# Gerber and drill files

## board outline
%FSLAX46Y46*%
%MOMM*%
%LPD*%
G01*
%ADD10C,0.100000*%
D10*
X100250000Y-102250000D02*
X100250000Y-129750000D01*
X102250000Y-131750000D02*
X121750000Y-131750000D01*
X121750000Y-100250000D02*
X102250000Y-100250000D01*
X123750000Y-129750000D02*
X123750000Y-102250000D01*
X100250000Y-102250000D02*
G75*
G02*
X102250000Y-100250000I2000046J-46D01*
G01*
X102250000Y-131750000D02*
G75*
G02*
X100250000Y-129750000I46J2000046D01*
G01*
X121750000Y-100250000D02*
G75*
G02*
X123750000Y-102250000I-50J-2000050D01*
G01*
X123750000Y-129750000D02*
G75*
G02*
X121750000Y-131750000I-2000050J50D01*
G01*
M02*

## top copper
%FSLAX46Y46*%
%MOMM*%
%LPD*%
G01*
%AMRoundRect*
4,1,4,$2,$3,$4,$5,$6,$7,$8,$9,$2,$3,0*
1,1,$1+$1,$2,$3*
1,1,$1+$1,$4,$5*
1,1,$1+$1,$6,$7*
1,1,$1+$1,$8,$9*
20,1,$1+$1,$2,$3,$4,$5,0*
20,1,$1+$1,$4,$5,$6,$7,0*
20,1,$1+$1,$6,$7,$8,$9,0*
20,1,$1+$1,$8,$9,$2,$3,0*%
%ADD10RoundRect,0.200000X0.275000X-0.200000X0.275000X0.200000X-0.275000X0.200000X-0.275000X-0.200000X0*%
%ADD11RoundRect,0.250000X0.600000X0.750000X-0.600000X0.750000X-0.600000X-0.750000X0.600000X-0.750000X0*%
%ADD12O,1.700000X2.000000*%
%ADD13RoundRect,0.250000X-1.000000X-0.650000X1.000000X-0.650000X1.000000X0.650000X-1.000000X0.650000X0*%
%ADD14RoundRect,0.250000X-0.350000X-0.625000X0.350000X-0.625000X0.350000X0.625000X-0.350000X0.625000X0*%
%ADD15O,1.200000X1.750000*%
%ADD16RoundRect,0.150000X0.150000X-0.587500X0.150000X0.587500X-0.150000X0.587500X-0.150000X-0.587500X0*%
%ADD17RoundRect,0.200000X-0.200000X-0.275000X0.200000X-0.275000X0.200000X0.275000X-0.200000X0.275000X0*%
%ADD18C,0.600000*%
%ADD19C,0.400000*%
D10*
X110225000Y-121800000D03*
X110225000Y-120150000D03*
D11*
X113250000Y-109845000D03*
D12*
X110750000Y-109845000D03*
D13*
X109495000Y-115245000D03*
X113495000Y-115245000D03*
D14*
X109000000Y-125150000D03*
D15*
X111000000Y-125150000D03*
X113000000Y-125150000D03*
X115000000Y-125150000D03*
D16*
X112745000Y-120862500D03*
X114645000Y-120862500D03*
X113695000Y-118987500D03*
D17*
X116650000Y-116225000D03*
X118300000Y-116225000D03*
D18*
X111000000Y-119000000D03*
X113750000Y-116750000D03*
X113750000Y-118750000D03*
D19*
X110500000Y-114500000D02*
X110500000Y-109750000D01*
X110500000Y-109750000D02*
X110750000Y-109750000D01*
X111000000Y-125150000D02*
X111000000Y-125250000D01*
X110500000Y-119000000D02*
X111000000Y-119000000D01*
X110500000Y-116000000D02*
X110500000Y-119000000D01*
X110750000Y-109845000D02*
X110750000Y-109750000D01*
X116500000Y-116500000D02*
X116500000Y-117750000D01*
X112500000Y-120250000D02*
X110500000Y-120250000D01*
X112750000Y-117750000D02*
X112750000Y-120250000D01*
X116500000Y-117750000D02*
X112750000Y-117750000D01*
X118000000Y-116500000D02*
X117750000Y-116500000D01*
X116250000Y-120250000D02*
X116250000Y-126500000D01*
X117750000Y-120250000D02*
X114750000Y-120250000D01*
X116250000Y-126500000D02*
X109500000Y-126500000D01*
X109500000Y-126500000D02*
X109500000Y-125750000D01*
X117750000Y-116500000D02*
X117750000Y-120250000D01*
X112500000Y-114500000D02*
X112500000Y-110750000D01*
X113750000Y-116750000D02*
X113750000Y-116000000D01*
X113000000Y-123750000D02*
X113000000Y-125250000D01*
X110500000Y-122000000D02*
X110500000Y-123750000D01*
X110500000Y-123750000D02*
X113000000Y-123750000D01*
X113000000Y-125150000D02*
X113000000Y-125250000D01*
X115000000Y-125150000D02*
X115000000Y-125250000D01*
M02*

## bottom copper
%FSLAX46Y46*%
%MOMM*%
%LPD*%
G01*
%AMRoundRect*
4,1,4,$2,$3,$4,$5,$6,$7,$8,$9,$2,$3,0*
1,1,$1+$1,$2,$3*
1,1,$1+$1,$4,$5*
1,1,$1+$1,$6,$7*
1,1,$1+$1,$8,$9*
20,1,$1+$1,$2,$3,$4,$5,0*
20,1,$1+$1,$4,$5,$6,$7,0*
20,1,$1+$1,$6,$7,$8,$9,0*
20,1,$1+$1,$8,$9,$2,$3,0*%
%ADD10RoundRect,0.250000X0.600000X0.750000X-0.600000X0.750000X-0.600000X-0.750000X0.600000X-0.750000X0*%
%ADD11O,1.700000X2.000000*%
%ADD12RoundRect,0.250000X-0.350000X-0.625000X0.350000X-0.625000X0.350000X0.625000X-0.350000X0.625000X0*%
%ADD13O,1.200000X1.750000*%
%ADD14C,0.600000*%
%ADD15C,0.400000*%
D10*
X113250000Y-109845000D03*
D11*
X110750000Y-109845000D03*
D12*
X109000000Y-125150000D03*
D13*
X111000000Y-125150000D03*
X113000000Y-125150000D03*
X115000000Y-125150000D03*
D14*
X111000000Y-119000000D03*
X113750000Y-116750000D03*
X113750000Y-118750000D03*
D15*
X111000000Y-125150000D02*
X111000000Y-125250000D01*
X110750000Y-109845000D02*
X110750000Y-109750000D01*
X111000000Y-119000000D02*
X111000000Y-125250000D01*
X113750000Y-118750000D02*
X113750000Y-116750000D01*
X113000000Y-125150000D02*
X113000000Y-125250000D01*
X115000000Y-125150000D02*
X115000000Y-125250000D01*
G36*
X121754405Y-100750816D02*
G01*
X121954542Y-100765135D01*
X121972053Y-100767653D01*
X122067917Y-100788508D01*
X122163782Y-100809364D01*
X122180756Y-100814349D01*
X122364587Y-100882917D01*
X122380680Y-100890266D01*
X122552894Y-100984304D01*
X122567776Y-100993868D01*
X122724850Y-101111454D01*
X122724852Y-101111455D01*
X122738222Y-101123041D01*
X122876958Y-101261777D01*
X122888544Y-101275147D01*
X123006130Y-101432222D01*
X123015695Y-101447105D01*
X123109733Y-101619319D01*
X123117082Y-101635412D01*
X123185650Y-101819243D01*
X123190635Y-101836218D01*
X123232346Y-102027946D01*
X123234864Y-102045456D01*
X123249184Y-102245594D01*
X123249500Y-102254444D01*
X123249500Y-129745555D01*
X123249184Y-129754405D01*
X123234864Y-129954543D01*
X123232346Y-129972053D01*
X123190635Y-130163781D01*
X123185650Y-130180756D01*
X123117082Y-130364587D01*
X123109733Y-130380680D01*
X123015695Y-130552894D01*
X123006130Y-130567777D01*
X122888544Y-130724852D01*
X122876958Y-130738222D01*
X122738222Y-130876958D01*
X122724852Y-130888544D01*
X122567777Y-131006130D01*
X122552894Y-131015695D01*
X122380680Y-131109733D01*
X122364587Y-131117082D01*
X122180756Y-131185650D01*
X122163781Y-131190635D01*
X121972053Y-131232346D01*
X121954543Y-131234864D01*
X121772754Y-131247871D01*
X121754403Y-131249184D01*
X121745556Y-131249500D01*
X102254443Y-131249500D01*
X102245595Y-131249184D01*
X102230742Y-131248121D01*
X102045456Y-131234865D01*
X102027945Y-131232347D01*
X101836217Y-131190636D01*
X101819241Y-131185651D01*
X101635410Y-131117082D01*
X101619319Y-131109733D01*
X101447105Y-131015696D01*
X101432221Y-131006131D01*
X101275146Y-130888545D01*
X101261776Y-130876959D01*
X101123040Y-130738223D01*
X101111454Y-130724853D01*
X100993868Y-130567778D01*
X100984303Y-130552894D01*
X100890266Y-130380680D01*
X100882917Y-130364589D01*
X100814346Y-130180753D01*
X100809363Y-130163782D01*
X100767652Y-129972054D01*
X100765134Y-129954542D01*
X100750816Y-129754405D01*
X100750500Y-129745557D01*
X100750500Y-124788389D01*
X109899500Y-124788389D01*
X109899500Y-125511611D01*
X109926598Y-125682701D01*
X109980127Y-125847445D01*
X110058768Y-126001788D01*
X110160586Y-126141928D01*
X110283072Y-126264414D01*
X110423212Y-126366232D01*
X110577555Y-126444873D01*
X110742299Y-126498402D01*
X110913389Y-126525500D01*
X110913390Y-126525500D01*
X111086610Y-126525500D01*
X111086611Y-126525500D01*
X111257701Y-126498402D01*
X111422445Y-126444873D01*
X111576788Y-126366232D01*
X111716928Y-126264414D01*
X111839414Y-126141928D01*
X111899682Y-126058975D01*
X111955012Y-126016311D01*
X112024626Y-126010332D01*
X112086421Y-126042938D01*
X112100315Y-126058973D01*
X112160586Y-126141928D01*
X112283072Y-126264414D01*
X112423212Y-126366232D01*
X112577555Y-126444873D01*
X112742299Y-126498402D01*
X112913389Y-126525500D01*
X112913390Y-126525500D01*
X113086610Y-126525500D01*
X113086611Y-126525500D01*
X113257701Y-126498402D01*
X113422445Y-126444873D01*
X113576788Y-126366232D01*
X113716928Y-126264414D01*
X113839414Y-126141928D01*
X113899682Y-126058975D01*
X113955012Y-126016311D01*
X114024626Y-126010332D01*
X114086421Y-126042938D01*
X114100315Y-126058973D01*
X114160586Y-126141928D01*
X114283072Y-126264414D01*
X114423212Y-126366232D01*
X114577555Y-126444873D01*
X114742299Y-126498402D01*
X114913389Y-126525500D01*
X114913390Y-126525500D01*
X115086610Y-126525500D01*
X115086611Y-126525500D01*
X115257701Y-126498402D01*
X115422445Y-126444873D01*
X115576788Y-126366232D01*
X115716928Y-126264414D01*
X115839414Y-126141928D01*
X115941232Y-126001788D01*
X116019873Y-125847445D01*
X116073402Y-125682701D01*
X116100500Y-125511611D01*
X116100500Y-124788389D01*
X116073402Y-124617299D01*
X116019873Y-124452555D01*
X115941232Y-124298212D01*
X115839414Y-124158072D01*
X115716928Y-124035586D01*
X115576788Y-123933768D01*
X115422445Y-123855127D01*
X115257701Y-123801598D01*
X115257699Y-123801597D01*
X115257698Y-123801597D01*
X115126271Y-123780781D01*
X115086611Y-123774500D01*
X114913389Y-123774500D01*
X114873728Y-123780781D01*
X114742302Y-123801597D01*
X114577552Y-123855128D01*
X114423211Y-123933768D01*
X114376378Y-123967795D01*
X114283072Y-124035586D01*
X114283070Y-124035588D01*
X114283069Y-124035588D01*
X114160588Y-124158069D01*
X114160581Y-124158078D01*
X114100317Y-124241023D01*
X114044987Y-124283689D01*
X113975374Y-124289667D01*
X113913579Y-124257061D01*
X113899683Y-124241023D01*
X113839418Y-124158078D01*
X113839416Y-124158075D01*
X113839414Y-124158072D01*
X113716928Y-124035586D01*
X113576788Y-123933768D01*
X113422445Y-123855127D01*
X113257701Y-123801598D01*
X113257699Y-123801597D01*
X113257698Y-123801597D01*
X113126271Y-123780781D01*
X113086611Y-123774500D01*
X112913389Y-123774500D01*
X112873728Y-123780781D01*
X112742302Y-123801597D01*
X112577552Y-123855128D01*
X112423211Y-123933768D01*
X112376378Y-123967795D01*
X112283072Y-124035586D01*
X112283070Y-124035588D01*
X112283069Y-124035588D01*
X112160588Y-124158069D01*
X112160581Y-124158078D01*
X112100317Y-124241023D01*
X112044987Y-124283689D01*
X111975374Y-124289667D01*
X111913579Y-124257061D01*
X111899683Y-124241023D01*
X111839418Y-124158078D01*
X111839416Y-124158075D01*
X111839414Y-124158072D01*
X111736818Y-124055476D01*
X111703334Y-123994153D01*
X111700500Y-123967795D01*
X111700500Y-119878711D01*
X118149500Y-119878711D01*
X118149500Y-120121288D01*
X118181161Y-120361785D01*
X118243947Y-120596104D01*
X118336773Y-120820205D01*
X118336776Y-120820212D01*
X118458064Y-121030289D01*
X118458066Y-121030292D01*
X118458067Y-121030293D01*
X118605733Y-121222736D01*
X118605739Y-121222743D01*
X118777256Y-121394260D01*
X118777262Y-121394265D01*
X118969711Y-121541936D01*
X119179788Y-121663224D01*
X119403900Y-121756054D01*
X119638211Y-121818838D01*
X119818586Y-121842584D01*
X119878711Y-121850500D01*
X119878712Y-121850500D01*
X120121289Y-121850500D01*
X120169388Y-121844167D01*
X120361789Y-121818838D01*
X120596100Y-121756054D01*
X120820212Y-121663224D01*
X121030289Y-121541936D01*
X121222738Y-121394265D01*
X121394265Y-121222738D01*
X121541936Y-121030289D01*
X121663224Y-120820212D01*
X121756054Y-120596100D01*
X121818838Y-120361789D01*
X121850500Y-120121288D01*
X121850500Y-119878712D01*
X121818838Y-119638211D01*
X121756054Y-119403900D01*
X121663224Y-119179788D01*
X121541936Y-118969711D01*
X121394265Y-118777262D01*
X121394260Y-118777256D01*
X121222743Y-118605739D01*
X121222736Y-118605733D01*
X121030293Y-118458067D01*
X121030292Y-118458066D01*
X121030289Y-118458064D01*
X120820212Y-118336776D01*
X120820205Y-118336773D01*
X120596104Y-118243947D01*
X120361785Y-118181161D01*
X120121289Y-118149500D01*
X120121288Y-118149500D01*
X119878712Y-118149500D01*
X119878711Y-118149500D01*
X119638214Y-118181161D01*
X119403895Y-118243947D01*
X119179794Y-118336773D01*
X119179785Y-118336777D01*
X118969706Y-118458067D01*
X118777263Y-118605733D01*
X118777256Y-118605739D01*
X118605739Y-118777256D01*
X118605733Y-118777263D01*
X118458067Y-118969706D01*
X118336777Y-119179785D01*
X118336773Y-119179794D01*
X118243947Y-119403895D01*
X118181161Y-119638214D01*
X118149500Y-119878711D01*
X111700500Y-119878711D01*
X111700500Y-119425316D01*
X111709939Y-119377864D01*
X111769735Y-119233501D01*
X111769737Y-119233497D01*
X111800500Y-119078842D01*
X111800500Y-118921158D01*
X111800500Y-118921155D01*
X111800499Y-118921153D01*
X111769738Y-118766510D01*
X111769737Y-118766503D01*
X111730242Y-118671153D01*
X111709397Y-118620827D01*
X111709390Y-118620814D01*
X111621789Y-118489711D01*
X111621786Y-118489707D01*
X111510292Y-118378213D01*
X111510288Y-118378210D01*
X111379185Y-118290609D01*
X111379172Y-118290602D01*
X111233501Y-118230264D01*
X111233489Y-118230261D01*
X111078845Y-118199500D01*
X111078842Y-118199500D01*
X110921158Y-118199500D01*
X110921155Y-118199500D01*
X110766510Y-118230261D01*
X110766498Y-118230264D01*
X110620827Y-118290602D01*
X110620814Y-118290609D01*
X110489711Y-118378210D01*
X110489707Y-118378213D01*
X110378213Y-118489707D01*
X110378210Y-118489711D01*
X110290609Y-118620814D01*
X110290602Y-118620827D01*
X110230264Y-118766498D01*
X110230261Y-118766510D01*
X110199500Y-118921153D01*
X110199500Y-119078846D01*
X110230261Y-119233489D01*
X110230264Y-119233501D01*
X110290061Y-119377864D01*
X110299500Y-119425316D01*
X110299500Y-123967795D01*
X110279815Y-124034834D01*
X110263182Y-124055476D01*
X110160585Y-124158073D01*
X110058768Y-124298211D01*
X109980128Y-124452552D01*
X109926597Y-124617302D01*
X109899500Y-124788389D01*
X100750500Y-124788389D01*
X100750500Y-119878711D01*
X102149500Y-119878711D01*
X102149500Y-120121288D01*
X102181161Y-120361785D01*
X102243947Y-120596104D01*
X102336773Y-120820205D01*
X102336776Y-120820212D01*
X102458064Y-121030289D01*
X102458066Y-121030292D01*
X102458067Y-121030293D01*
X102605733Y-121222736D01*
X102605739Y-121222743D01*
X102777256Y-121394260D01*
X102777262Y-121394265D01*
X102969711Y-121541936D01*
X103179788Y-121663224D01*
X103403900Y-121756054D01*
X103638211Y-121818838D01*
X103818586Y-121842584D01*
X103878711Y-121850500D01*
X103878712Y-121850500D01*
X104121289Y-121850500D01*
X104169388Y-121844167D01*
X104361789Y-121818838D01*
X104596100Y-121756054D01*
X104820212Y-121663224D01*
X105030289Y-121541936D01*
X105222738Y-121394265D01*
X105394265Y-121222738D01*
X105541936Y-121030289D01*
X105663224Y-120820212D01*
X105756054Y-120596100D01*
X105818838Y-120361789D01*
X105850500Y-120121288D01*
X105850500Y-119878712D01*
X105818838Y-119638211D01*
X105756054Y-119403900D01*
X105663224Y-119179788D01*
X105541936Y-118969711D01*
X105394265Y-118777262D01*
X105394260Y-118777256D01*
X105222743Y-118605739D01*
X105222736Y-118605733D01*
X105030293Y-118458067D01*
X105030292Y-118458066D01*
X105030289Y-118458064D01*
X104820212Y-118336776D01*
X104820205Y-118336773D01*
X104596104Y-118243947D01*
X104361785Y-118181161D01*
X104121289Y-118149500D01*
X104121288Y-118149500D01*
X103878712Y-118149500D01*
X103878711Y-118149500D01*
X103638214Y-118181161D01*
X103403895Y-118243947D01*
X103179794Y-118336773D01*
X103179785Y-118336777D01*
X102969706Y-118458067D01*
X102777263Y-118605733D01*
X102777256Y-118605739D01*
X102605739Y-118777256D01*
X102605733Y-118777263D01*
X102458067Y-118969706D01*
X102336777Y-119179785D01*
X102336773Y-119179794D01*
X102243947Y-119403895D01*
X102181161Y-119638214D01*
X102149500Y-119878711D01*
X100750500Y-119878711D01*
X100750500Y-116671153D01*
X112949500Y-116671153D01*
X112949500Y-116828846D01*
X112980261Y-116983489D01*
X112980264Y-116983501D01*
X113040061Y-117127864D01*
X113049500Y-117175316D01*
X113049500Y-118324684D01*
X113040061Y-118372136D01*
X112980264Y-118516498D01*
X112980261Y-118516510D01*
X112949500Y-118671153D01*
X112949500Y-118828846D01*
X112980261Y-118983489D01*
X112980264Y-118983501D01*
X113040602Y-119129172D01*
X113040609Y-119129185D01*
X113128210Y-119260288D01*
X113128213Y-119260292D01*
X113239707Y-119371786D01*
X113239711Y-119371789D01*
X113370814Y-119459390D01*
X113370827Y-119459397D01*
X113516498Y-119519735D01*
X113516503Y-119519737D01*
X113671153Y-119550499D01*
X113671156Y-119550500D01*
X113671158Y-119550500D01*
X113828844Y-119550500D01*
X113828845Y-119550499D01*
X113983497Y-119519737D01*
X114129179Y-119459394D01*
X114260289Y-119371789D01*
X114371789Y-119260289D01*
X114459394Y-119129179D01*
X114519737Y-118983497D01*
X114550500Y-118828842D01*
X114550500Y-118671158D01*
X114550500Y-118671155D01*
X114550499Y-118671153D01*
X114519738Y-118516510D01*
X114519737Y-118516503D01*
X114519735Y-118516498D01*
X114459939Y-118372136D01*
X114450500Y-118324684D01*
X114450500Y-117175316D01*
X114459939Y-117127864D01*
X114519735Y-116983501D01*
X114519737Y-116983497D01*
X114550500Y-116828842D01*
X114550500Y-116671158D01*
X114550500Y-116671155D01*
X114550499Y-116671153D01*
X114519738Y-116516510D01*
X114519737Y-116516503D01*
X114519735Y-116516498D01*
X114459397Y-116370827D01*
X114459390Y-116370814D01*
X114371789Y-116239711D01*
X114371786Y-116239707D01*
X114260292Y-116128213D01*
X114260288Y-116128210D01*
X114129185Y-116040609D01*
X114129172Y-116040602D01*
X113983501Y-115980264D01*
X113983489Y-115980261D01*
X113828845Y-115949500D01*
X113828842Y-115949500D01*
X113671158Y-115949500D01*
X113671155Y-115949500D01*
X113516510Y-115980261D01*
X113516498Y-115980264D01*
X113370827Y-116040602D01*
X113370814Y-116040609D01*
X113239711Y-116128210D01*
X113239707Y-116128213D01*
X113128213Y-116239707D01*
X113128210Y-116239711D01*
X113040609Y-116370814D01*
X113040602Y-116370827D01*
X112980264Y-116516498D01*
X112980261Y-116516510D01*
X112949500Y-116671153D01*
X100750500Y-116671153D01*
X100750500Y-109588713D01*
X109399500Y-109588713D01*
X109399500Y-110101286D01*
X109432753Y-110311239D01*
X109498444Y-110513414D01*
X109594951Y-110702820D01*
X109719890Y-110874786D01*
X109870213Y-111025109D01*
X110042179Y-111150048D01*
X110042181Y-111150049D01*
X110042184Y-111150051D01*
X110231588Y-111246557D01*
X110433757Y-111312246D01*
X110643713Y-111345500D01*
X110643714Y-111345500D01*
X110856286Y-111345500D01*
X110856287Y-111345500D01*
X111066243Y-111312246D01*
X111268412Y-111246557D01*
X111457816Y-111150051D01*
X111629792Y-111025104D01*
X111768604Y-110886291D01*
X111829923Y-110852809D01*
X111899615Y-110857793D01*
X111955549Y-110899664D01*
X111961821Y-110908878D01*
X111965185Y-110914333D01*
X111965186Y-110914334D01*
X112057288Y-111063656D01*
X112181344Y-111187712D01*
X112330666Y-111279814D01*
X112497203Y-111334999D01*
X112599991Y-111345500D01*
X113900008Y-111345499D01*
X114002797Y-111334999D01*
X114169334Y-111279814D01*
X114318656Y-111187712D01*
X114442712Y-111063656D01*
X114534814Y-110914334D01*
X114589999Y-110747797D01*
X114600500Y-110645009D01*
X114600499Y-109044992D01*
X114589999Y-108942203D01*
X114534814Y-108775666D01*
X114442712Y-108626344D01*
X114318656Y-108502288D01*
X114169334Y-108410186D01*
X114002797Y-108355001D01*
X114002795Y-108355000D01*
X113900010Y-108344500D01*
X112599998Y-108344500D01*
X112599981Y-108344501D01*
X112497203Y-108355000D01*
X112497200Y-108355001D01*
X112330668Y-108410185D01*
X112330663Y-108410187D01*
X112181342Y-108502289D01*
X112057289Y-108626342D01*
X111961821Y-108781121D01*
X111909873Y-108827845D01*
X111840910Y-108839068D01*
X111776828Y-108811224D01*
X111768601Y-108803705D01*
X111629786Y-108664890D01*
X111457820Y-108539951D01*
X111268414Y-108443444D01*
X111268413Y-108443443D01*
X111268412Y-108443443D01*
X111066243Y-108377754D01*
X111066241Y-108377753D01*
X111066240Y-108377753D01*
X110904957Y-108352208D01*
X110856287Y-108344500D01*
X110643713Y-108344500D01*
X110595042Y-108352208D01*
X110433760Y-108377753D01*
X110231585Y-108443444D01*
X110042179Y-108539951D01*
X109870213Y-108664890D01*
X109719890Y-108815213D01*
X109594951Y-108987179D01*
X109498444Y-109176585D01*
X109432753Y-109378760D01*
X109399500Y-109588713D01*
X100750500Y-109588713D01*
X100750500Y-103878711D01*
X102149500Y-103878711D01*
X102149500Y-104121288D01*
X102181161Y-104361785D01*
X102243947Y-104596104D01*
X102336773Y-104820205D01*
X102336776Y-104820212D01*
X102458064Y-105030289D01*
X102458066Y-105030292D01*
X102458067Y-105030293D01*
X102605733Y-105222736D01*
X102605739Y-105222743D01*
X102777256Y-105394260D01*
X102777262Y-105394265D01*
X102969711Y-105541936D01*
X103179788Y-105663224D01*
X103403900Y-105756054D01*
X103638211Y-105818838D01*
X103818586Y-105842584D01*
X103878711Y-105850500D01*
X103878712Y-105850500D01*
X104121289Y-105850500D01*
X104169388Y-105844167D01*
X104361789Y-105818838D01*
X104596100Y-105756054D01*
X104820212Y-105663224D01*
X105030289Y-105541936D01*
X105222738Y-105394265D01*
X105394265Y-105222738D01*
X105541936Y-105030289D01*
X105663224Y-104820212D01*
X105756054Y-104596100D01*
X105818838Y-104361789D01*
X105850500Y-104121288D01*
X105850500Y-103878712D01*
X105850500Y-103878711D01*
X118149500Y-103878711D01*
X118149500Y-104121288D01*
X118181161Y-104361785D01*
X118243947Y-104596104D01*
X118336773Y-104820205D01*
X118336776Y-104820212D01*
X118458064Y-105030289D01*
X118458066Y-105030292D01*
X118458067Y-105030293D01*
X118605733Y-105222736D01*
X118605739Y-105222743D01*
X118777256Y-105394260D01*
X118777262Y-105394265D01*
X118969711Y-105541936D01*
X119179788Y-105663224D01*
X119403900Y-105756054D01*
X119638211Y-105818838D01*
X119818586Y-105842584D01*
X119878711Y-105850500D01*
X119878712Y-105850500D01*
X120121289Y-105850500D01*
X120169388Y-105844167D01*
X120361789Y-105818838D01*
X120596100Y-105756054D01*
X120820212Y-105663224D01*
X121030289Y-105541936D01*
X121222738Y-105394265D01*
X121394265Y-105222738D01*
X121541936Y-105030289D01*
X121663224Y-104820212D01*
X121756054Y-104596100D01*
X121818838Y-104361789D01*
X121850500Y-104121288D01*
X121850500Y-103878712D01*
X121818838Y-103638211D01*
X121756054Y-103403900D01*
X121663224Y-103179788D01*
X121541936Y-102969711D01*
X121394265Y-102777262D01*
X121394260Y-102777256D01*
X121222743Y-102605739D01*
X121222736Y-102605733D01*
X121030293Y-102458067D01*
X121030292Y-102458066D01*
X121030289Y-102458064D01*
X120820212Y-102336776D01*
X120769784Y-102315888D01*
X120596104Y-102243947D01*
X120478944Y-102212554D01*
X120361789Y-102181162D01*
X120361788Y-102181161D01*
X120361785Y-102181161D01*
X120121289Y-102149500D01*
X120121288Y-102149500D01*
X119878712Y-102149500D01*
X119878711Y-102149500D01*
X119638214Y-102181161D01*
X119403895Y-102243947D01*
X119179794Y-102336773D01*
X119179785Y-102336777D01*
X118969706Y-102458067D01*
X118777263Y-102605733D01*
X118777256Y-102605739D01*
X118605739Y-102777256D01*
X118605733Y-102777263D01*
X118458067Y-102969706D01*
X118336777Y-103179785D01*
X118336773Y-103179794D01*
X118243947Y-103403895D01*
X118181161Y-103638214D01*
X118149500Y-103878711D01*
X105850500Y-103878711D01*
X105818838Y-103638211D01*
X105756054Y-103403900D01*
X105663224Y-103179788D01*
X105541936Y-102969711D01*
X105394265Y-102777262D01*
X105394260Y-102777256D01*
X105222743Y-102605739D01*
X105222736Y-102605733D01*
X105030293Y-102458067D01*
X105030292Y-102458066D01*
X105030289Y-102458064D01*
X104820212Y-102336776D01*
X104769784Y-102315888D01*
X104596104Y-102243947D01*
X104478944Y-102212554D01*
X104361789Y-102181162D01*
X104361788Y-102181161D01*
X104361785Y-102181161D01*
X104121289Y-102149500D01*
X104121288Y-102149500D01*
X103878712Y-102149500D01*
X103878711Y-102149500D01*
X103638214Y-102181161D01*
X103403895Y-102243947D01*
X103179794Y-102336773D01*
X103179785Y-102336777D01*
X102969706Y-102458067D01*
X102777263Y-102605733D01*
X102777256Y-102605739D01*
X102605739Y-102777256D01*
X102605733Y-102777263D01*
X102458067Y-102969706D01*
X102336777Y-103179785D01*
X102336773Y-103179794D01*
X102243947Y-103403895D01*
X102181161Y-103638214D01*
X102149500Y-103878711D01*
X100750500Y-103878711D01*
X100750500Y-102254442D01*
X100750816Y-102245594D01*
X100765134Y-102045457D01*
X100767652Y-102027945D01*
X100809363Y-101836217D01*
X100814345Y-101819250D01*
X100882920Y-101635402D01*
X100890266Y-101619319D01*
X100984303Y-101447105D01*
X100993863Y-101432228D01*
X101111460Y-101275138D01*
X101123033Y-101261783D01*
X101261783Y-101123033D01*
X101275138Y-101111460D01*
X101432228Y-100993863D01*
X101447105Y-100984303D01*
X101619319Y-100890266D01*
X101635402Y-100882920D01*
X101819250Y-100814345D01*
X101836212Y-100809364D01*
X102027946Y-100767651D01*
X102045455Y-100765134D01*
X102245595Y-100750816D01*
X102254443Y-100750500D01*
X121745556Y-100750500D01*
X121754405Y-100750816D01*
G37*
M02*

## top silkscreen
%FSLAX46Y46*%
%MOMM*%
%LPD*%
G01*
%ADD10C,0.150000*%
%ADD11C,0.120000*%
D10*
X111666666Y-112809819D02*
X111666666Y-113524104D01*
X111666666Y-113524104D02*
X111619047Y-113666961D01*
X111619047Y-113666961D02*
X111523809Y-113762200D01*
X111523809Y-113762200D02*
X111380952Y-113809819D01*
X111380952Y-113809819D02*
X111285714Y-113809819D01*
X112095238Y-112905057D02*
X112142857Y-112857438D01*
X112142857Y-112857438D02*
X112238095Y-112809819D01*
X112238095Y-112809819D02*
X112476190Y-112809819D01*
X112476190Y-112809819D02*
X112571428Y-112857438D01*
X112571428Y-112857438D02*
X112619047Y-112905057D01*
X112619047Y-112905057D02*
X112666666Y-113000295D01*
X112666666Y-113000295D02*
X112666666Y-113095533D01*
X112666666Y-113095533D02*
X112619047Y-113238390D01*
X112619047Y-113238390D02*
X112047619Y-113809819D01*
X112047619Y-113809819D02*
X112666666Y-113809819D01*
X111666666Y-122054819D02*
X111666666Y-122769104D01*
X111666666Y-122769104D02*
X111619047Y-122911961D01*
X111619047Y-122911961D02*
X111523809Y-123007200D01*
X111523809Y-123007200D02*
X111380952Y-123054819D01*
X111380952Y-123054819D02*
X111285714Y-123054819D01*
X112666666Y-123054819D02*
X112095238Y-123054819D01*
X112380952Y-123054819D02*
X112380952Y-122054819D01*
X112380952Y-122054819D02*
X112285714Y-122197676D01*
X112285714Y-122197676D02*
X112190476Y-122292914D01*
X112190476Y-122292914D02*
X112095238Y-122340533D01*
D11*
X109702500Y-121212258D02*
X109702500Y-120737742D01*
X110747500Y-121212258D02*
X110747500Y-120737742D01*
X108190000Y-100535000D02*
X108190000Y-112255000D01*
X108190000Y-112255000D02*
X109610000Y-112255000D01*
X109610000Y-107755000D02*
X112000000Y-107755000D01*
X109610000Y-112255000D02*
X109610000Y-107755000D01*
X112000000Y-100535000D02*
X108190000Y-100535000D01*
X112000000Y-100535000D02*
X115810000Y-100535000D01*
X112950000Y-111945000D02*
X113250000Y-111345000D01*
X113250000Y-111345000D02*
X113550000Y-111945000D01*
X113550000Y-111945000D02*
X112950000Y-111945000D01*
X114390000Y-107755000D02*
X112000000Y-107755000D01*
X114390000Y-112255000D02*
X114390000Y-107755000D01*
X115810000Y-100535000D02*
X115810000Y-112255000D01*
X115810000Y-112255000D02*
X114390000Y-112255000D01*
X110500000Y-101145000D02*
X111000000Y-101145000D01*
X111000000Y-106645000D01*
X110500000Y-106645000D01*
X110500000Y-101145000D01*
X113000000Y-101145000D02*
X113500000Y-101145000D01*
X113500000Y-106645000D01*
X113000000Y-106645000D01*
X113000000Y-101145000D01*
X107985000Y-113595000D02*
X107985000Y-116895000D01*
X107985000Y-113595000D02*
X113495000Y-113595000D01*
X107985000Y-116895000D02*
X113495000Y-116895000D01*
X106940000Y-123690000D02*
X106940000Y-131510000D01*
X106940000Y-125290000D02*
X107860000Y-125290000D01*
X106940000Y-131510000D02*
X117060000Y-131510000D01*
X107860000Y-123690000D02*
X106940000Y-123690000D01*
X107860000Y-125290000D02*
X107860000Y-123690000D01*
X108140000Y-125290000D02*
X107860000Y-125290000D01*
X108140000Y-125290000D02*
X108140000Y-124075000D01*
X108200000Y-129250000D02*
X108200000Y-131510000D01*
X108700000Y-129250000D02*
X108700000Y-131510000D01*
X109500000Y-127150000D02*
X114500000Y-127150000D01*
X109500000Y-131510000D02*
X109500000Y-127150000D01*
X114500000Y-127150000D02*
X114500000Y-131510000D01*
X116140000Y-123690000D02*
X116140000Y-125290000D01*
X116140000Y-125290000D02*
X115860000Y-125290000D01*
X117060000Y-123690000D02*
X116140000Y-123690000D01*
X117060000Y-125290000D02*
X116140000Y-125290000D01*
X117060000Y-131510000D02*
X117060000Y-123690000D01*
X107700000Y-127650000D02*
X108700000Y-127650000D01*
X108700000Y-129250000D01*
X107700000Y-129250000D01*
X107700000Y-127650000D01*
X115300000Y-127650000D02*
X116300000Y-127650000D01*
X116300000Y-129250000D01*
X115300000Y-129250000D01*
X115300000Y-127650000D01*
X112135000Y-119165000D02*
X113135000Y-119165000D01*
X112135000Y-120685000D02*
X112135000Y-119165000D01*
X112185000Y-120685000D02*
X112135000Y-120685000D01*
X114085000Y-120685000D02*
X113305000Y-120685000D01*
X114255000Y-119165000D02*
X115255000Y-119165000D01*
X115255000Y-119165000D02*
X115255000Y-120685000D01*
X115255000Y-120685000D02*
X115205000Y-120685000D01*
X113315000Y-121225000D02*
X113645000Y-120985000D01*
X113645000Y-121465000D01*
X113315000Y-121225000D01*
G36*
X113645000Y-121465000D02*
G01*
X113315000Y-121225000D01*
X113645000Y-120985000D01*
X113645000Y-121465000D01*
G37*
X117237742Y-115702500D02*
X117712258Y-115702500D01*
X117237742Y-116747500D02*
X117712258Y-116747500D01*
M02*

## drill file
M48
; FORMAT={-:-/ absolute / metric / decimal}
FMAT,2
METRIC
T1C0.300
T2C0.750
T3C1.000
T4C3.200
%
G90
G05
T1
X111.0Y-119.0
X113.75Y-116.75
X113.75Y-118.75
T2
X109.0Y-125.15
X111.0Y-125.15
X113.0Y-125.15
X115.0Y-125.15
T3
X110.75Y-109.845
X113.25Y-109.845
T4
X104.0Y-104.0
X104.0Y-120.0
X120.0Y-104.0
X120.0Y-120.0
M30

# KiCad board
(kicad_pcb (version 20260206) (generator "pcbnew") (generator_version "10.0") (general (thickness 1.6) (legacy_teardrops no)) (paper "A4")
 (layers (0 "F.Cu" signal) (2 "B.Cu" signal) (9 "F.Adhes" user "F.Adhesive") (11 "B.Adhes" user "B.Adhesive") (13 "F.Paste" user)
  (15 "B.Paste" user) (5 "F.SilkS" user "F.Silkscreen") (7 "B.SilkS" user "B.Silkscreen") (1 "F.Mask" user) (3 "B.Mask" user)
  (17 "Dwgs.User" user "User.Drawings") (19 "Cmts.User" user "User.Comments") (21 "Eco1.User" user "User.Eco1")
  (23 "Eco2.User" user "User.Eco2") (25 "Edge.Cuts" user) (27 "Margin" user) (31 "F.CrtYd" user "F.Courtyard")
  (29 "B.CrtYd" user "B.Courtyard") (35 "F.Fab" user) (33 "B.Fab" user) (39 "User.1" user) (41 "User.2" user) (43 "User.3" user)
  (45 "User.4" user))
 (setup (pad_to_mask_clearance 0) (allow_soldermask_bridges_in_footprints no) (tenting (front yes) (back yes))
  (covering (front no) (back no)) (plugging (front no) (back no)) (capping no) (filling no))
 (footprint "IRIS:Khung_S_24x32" (layer "F.Cu") (at 100 132)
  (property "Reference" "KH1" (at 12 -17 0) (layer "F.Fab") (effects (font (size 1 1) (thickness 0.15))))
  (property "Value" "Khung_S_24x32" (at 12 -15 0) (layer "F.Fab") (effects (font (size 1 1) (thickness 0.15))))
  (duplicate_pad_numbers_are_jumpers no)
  (fp_line (start 0.25 -29.75) (end 0.25 -2.25) (stroke (width 0.1) (type solid)) (layer "Edge.Cuts"))
  (fp_line (start 2.25 -0.25) (end 21.75 -0.25) (stroke (width 0.1) (type solid)) (layer "Edge.Cuts"))
  (fp_line (start 21.75 -31.75) (end 2.25 -31.75) (stroke (width 0.1) (type solid)) (layer "Edge.Cuts"))
  (fp_line (start 23.75 -2.25) (end 23.75 -29.75) (stroke (width 0.1) (type solid)) (layer "Edge.Cuts"))
  (fp_arc (start 0.25 -29.75) (mid 0.8358 -31.1642) (end 2.25 -31.75) (stroke (width 0.1) (type solid)) (layer "Edge.Cuts"))
  (fp_arc (start 2.25 -0.25) (mid 0.8358 -0.8358) (end 0.25 -2.25) (stroke (width 0.1) (type solid)) (layer "Edge.Cuts"))
  (fp_arc (start 21.75 -31.75) (mid 23.164199 -31.164199) (end 23.75 -29.75) (stroke (width 0.1) (type solid)) (layer "Edge.Cuts"))
  (fp_arc (start 23.75 -2.25) (mid 23.164199 -0.835801) (end 21.75 -0.25) (stroke (width 0.1) (type solid)) (layer "Edge.Cuts"))
  (pad "" np_thru_hole circle (at 4 -28) (size 3.2 3.2) (drill 3.2) (layers "*.Cu" "*.Mask"))
  (pad "" np_thru_hole circle (at 4 -12) (size 3.2 3.2) (drill 3.2) (layers "*.Cu" "*.Mask"))
  (pad "" np_thru_hole circle (at 20 -28) (size 3.2 3.2) (drill 3.2) (layers "*.Cu" "*.Mask"))
  (pad "" np_thru_hole circle (at 20 -12) (size 3.2 3.2) (drill 3.2) (layers "*.Cu" "*.Mask")))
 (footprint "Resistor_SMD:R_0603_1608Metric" (layer "F.Cu") (at 110.225 120.975 90)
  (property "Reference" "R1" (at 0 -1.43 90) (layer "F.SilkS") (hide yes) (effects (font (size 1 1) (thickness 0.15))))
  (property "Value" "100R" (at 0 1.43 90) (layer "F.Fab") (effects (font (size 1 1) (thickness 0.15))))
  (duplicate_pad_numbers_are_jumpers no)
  (fp_line (start -0.237258 -0.5225) (end 0.237258 -0.5225) (stroke (width 0.12) (type solid)) (layer "F.SilkS"))
  (fp_line (start -0.237258 0.5225) (end 0.237258 0.5225) (stroke (width 0.12) (type solid)) (layer "F.SilkS"))
  (pad "1" smd roundrect (at -0.825 0 90) (size 0.8 0.95) (layers "F.Cu" "F.Mask" "F.Paste") (roundrect_rratio 0.25) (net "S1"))
  (pad "2" smd roundrect (at 0.825 0 90) (size 0.8 0.95) (layers "F.Cu" "F.Mask" "F.Paste") (roundrect_rratio 0.25) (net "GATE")))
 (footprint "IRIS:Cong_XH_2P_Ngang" (layer "F.Cu") (at 113.25 109.845 180)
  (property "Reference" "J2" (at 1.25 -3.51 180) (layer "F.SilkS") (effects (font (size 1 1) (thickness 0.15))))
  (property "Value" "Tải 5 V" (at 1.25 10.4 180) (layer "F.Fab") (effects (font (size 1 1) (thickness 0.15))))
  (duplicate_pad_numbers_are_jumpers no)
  (fp_line (start 5.06 9.31) (end 5.06 -2.41) (stroke (width 0.12) (type solid)) (layer "F.SilkS"))
  (fp_line (start 5.06 -2.41) (end 3.64 -2.41) (stroke (width 0.12) (type solid)) (layer "F.SilkS"))
  (fp_line (start 3.64 2.09) (end 1.25 2.09) (stroke (width 0.12) (type solid)) (layer "F.SilkS"))
  (fp_line (start 3.64 -2.41) (end 3.64 2.09) (stroke (width 0.12) (type solid)) (layer "F.SilkS"))
  (fp_line (start 1.25 9.31) (end 5.06 9.31) (stroke (width 0.12) (type solid)) (layer "F.SilkS"))
  (fp_line (start 1.25 9.31) (end -2.56 9.31) (stroke (width 0.12) (type solid)) (layer "F.SilkS"))
  (fp_line (start 0.3 -2.1) (end 0 -1.5) (stroke (width 0.12) (type solid)) (layer "F.SilkS"))
  (fp_line (start 0 -1.5) (end -0.3 -2.1) (stroke (width 0.12) (type solid)) (layer "F.SilkS"))
  (fp_line (start -0.3 -2.1) (end 0.3 -2.1) (stroke (width 0.12) (type solid)) (layer "F.SilkS"))
  (fp_line (start -1.14 2.09) (end 1.25 2.09) (stroke (width 0.12) (type solid)) (layer "F.SilkS"))
  (fp_line (start -1.14 -2.41) (end -1.14 2.09) (stroke (width 0.12) (type solid)) (layer "F.SilkS"))
  (fp_line (start -2.56 9.31) (end -2.56 -2.41) (stroke (width 0.12) (type solid)) (layer "F.SilkS"))
  (fp_line (start -2.56 -2.41) (end -1.14 -2.41) (stroke (width 0.12) (type solid)) (layer "F.SilkS"))
  (fp_rect (start 2.25 3.2) (end 2.75 8.7) (stroke (width 0.12) (type solid)) (fill no) (layer "F.SilkS"))
  (fp_rect (start -0.25 3.2) (end 0.25 8.7) (stroke (width 0.12) (type solid)) (fill no) (layer "F.SilkS"))
  (pad "1" thru_hole roundrect (at 0 0 180) (size 1.7 2) (drill 1) (layers "*.Cu" "*.Mask") (remove_unused_layers no)
   (roundrect_rratio 0.147059) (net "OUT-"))
  (pad "2" thru_hole oval (at 2.5 0 180) (size 1.7 2) (drill 1) (layers "*.Cu" "*.Mask") (remove_unused_layers no) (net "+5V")))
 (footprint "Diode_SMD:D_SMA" (layer "F.Cu") (at 111.495 115.245)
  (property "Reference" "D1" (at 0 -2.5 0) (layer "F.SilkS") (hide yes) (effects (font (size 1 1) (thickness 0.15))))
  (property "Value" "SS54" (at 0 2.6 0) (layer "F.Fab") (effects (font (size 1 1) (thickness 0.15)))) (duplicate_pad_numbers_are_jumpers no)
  (fp_line (start -3.51 -1.65) (end -3.51 1.65) (stroke (width 0.12) (type solid)) (layer "F.SilkS"))
  (fp_line (start -3.51 -1.65) (end 2 -1.65) (stroke (width 0.12) (type solid)) (layer "F.SilkS"))
  (fp_line (start -3.51 1.65) (end 2 1.65) (stroke (width 0.12) (type solid)) (layer "F.SilkS"))
  (pad "1" smd roundrect (at -2 0) (size 2.5 1.8) (layers "F.Cu" "F.Mask" "F.Paste") (roundrect_rratio 0.1388888889) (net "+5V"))
  (pad "2" smd roundrect (at 2 0) (size 2.5 1.8) (layers "F.Cu" "F.Mask" "F.Paste") (roundrect_rratio 0.1388888889) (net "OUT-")))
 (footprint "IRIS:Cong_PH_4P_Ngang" (layer "F.Cu") (at 109 125.15)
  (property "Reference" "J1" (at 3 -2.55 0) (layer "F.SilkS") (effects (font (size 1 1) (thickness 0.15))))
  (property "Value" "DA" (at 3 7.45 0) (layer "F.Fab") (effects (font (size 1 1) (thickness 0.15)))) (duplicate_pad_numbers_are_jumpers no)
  (fp_line (start -2.06 -1.46) (end -2.06 6.36) (stroke (width 0.12) (type solid)) (layer "F.SilkS"))
  (fp_line (start -2.06 0.14) (end -1.14 0.14) (stroke (width 0.12) (type solid)) (layer "F.SilkS"))
  (fp_line (start -2.06 6.36) (end 8.06 6.36) (stroke (width 0.12) (type solid)) (layer "F.SilkS"))
  (fp_line (start -1.14 -1.46) (end -2.06 -1.46) (stroke (width 0.12) (type solid)) (layer "F.SilkS"))
  (fp_line (start -1.14 0.14) (end -1.14 -1.46) (stroke (width 0.12) (type solid)) (layer "F.SilkS"))
  (fp_line (start -0.86 0.14) (end -1.14 0.14) (stroke (width 0.12) (type solid)) (layer "F.SilkS"))
  (fp_line (start -0.86 0.14) (end -0.86 -1.075) (stroke (width 0.12) (type solid)) (layer "F.SilkS"))
  (fp_line (start -0.8 4.1) (end -0.8 6.36) (stroke (width 0.12) (type solid)) (layer "F.SilkS"))
  (fp_line (start -0.3 4.1) (end -0.3 6.36) (stroke (width 0.12) (type solid)) (layer "F.SilkS"))
  (fp_line (start 0.5 2) (end 5.5 2) (stroke (width 0.12) (type solid)) (layer "F.SilkS"))
  (fp_line (start 0.5 6.36) (end 0.5 2) (stroke (width 0.12) (type solid)) (layer "F.SilkS"))
  (fp_line (start 5.5 2) (end 5.5 6.36) (stroke (width 0.12) (type solid)) (layer "F.SilkS"))
  (fp_line (start 7.14 -1.46) (end 7.14 0.14) (stroke (width 0.12) (type solid)) (layer "F.SilkS"))
  (fp_line (start 7.14 0.14) (end 6.86 0.14) (stroke (width 0.12) (type solid)) (layer "F.SilkS"))
  (fp_line (start 8.06 -1.46) (end 7.14 -1.46) (stroke (width 0.12) (type solid)) (layer "F.SilkS"))
  (fp_line (start 8.06 0.14) (end 7.14 0.14) (stroke (width 0.12) (type solid)) (layer "F.SilkS"))
  (fp_line (start 8.06 6.36) (end 8.06 -1.46) (stroke (width 0.12) (type solid)) (layer "F.SilkS"))
  (fp_rect (start -1.3 2.5) (end -0.3 4.1) (stroke (width 0.12) (type solid)) (fill no) (layer "F.SilkS"))
  (fp_rect (start 6.3 2.5) (end 7.3 4.1) (stroke (width 0.12) (type solid)) (fill no) (layer "F.SilkS"))
  (pad "1" thru_hole roundrect (at 0 0) (size 1.2 1.75) (drill 0.75) (layers "*.Cu" "*.Mask") (remove_unused_layers no)
   (roundrect_rratio 0.208333) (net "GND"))
  (pad "2" thru_hole oval (at 2 0) (size 1.2 1.75) (drill 0.75) (layers "*.Cu" "*.Mask") (remove_unused_layers no) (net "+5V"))
  (pad "3" thru_hole oval (at 4 0) (size 1.2 1.75) (drill 0.75) (layers "*.Cu" "*.Mask") (remove_unused_layers no) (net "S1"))
  (pad "4" thru_hole oval (at 6 0) (size 1.2 1.75) (drill 0.75) (layers "*.Cu" "*.Mask") (remove_unused_layers no)
   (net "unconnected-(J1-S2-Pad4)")))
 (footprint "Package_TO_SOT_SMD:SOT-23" (layer "F.Cu") (at 113.695 119.925 90)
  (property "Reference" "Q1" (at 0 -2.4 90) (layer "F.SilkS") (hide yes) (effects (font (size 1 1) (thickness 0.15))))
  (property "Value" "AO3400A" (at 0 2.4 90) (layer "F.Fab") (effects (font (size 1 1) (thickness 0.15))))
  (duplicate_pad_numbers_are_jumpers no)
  (fp_line (start 0.76 -1.56) (end 0.76 -0.56) (stroke (width 0.12) (type solid)) (layer "F.SilkS"))
  (fp_line (start -0.76 -1.56) (end 0.76 -1.56) (stroke (width 0.12) (type solid)) (layer "F.SilkS"))
  (fp_line (start -0.76 -1.51) (end -0.76 -1.56) (stroke (width 0.12) (type solid)) (layer "F.SilkS"))
  (fp_line (start -0.76 0.39) (end -0.76 -0.39) (stroke (width 0.12) (type solid)) (layer "F.SilkS"))
  (fp_line (start 0.76 0.56) (end 0.76 1.56) (stroke (width 0.12) (type solid)) (layer "F.SilkS"))
  (fp_line (start 0.76 1.56) (end -0.76 1.56) (stroke (width 0.12) (type solid)) (layer "F.SilkS"))
  (fp_line (start -0.76 1.56) (end -0.76 1.51) (stroke (width 0.12) (type solid)) (layer "F.SilkS"))
  (fp_poly (pts (xy -1.3 -0.38) (xy -1.06 -0.05) (xy -1.54 -0.05)) (stroke (width 0.12) (type solid)) (fill yes) (layer "F.SilkS"))
  (pad "1" smd roundrect (at -0.9375 -0.95 90) (size 1.475 0.6) (layers "F.Cu" "F.Mask" "F.Paste") (roundrect_rratio 0.25) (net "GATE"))
  (pad "2" smd roundrect (at -0.9375 0.95 90) (size 1.475 0.6) (layers "F.Cu" "F.Mask" "F.Paste") (roundrect_rratio 0.25) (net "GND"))
  (pad "3" smd roundrect (at 0.9375 0 90) (size 1.475 0.6) (layers "F.Cu" "F.Mask" "F.Paste") (roundrect_rratio 0.25) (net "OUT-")))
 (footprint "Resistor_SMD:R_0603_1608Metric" (layer "F.Cu") (at 117.475 116.225)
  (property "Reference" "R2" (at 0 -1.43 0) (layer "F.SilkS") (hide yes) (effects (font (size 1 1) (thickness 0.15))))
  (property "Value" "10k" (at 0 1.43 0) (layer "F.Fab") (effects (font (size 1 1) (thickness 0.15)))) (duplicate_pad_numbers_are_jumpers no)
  (fp_line (start -0.237258 -0.5225) (end 0.237258 -0.5225) (stroke (width 0.12) (type solid)) (layer "F.SilkS"))
  (fp_line (start -0.237258 0.5225) (end 0.237258 0.5225) (stroke (width 0.12) (type solid)) (layer "F.SilkS"))
  (pad "1" smd roundrect (at -0.825 0) (size 0.8 0.95) (layers "F.Cu" "F.Mask" "F.Paste") (roundrect_rratio 0.25) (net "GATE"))
  (pad "2" smd roundrect (at 0.825 0) (size 0.8 0.95) (layers "F.Cu" "F.Mask" "F.Paste") (roundrect_rratio 0.25) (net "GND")))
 (segment (start 110.5 114.5) (end 110.5 109.75) (width 0.4) (layer "F.Cu") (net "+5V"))
 (segment (start 110.5 109.75) (end 110.75 109.75) (width 0.4) (layer "F.Cu") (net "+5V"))
 (segment (start 111 125.15) (end 111 125.25) (width 0.4) (layer "F.Cu") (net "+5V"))
 (segment (start 110.5 119) (end 111 119) (width 0.4) (layer "F.Cu") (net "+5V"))
 (segment (start 110.5 116) (end 110.5 119) (width 0.4) (layer "F.Cu") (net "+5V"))
 (segment (start 110.75 109.845) (end 110.75 109.75) (width 0.4) (layer "F.Cu") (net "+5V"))
 (via (at 111 119) (size 0.6) (drill 0.3) (layers "F.Cu" "B.Cu") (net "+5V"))
 (segment (start 111 125.15) (end 111 125.25) (width 0.4) (layer "B.Cu") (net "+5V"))
 (segment (start 110.75 109.845) (end 110.75 109.75) (width 0.4) (layer "B.Cu") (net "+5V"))
 (segment (start 111 119) (end 111 125.25) (width 0.4) (layer "B.Cu") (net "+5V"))
 (segment (start 116.5 116.5) (end 116.5 117.75) (width 0.4) (layer "F.Cu") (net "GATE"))
 (segment (start 112.5 120.25) (end 110.5 120.25) (width 0.4) (layer "F.Cu") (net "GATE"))
 (segment (start 112.75 117.75) (end 112.75 120.25) (width 0.4) (layer "F.Cu") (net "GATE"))
 (segment (start 116.5 117.75) (end 112.75 117.75) (width 0.4) (layer "F.Cu") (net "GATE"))
 (segment (start 118 116.5) (end 117.75 116.5) (width 0.4) (layer "F.Cu") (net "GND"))
 (segment (start 116.25 120.25) (end 116.25 126.5) (width 0.4) (layer "F.Cu") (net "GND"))
 (segment (start 117.75 120.25) (end 114.75 120.25) (width 0.4) (layer "F.Cu") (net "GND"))
 (segment (start 116.25 126.5) (end 109.5 126.5) (width 0.4) (layer "F.Cu") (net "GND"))
 (segment (start 109.5 126.5) (end 109.5 125.75) (width 0.4) (layer "F.Cu") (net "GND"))
 (segment (start 117.75 116.5) (end 117.75 120.25) (width 0.4) (layer "F.Cu") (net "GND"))
 (segment (start 112.5 114.5) (end 112.5 110.75) (width 0.4) (layer "F.Cu") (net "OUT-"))
 (segment (start 113.75 116.75) (end 113.75 116) (width 0.4) (layer "F.Cu") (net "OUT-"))
 (via (at 113.75 116.75) (size 0.6) (drill 0.3) (layers "F.Cu" "B.Cu") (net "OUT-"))
 (via (at 113.75 118.75) (size 0.6) (drill 0.3) (layers "F.Cu" "B.Cu") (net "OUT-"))
 (segment (start 113.75 118.75) (end 113.75 116.75) (width 0.4) (layer "B.Cu") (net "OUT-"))
 (segment (start 113 123.75) (end 113 125.25) (width 0.4) (layer "F.Cu") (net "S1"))
 (segment (start 110.5 122) (end 110.5 123.75) (width 0.4) (layer "F.Cu") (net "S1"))
 (segment (start 110.5 123.75) (end 113 123.75) (width 0.4) (layer "F.Cu") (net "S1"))
 (segment (start 113 125.15) (end 113 125.25) (width 0.4) (layer "F.Cu") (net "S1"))
 (segment (start 113 125.15) (end 113 125.25) (width 0.4) (layer "B.Cu") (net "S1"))
 (segment (start 115 125.15) (end 115 125.25) (width 0.4) (layer "F.Cu") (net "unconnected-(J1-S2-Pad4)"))
 (segment (start 115 125.15) (end 115 125.25) (width 0.4) (layer "B.Cu") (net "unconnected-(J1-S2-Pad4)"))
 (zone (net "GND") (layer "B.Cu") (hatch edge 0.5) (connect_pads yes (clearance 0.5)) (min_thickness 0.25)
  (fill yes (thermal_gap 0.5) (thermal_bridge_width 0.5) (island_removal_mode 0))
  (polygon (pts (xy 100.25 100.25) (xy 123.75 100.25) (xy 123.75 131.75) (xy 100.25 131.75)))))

